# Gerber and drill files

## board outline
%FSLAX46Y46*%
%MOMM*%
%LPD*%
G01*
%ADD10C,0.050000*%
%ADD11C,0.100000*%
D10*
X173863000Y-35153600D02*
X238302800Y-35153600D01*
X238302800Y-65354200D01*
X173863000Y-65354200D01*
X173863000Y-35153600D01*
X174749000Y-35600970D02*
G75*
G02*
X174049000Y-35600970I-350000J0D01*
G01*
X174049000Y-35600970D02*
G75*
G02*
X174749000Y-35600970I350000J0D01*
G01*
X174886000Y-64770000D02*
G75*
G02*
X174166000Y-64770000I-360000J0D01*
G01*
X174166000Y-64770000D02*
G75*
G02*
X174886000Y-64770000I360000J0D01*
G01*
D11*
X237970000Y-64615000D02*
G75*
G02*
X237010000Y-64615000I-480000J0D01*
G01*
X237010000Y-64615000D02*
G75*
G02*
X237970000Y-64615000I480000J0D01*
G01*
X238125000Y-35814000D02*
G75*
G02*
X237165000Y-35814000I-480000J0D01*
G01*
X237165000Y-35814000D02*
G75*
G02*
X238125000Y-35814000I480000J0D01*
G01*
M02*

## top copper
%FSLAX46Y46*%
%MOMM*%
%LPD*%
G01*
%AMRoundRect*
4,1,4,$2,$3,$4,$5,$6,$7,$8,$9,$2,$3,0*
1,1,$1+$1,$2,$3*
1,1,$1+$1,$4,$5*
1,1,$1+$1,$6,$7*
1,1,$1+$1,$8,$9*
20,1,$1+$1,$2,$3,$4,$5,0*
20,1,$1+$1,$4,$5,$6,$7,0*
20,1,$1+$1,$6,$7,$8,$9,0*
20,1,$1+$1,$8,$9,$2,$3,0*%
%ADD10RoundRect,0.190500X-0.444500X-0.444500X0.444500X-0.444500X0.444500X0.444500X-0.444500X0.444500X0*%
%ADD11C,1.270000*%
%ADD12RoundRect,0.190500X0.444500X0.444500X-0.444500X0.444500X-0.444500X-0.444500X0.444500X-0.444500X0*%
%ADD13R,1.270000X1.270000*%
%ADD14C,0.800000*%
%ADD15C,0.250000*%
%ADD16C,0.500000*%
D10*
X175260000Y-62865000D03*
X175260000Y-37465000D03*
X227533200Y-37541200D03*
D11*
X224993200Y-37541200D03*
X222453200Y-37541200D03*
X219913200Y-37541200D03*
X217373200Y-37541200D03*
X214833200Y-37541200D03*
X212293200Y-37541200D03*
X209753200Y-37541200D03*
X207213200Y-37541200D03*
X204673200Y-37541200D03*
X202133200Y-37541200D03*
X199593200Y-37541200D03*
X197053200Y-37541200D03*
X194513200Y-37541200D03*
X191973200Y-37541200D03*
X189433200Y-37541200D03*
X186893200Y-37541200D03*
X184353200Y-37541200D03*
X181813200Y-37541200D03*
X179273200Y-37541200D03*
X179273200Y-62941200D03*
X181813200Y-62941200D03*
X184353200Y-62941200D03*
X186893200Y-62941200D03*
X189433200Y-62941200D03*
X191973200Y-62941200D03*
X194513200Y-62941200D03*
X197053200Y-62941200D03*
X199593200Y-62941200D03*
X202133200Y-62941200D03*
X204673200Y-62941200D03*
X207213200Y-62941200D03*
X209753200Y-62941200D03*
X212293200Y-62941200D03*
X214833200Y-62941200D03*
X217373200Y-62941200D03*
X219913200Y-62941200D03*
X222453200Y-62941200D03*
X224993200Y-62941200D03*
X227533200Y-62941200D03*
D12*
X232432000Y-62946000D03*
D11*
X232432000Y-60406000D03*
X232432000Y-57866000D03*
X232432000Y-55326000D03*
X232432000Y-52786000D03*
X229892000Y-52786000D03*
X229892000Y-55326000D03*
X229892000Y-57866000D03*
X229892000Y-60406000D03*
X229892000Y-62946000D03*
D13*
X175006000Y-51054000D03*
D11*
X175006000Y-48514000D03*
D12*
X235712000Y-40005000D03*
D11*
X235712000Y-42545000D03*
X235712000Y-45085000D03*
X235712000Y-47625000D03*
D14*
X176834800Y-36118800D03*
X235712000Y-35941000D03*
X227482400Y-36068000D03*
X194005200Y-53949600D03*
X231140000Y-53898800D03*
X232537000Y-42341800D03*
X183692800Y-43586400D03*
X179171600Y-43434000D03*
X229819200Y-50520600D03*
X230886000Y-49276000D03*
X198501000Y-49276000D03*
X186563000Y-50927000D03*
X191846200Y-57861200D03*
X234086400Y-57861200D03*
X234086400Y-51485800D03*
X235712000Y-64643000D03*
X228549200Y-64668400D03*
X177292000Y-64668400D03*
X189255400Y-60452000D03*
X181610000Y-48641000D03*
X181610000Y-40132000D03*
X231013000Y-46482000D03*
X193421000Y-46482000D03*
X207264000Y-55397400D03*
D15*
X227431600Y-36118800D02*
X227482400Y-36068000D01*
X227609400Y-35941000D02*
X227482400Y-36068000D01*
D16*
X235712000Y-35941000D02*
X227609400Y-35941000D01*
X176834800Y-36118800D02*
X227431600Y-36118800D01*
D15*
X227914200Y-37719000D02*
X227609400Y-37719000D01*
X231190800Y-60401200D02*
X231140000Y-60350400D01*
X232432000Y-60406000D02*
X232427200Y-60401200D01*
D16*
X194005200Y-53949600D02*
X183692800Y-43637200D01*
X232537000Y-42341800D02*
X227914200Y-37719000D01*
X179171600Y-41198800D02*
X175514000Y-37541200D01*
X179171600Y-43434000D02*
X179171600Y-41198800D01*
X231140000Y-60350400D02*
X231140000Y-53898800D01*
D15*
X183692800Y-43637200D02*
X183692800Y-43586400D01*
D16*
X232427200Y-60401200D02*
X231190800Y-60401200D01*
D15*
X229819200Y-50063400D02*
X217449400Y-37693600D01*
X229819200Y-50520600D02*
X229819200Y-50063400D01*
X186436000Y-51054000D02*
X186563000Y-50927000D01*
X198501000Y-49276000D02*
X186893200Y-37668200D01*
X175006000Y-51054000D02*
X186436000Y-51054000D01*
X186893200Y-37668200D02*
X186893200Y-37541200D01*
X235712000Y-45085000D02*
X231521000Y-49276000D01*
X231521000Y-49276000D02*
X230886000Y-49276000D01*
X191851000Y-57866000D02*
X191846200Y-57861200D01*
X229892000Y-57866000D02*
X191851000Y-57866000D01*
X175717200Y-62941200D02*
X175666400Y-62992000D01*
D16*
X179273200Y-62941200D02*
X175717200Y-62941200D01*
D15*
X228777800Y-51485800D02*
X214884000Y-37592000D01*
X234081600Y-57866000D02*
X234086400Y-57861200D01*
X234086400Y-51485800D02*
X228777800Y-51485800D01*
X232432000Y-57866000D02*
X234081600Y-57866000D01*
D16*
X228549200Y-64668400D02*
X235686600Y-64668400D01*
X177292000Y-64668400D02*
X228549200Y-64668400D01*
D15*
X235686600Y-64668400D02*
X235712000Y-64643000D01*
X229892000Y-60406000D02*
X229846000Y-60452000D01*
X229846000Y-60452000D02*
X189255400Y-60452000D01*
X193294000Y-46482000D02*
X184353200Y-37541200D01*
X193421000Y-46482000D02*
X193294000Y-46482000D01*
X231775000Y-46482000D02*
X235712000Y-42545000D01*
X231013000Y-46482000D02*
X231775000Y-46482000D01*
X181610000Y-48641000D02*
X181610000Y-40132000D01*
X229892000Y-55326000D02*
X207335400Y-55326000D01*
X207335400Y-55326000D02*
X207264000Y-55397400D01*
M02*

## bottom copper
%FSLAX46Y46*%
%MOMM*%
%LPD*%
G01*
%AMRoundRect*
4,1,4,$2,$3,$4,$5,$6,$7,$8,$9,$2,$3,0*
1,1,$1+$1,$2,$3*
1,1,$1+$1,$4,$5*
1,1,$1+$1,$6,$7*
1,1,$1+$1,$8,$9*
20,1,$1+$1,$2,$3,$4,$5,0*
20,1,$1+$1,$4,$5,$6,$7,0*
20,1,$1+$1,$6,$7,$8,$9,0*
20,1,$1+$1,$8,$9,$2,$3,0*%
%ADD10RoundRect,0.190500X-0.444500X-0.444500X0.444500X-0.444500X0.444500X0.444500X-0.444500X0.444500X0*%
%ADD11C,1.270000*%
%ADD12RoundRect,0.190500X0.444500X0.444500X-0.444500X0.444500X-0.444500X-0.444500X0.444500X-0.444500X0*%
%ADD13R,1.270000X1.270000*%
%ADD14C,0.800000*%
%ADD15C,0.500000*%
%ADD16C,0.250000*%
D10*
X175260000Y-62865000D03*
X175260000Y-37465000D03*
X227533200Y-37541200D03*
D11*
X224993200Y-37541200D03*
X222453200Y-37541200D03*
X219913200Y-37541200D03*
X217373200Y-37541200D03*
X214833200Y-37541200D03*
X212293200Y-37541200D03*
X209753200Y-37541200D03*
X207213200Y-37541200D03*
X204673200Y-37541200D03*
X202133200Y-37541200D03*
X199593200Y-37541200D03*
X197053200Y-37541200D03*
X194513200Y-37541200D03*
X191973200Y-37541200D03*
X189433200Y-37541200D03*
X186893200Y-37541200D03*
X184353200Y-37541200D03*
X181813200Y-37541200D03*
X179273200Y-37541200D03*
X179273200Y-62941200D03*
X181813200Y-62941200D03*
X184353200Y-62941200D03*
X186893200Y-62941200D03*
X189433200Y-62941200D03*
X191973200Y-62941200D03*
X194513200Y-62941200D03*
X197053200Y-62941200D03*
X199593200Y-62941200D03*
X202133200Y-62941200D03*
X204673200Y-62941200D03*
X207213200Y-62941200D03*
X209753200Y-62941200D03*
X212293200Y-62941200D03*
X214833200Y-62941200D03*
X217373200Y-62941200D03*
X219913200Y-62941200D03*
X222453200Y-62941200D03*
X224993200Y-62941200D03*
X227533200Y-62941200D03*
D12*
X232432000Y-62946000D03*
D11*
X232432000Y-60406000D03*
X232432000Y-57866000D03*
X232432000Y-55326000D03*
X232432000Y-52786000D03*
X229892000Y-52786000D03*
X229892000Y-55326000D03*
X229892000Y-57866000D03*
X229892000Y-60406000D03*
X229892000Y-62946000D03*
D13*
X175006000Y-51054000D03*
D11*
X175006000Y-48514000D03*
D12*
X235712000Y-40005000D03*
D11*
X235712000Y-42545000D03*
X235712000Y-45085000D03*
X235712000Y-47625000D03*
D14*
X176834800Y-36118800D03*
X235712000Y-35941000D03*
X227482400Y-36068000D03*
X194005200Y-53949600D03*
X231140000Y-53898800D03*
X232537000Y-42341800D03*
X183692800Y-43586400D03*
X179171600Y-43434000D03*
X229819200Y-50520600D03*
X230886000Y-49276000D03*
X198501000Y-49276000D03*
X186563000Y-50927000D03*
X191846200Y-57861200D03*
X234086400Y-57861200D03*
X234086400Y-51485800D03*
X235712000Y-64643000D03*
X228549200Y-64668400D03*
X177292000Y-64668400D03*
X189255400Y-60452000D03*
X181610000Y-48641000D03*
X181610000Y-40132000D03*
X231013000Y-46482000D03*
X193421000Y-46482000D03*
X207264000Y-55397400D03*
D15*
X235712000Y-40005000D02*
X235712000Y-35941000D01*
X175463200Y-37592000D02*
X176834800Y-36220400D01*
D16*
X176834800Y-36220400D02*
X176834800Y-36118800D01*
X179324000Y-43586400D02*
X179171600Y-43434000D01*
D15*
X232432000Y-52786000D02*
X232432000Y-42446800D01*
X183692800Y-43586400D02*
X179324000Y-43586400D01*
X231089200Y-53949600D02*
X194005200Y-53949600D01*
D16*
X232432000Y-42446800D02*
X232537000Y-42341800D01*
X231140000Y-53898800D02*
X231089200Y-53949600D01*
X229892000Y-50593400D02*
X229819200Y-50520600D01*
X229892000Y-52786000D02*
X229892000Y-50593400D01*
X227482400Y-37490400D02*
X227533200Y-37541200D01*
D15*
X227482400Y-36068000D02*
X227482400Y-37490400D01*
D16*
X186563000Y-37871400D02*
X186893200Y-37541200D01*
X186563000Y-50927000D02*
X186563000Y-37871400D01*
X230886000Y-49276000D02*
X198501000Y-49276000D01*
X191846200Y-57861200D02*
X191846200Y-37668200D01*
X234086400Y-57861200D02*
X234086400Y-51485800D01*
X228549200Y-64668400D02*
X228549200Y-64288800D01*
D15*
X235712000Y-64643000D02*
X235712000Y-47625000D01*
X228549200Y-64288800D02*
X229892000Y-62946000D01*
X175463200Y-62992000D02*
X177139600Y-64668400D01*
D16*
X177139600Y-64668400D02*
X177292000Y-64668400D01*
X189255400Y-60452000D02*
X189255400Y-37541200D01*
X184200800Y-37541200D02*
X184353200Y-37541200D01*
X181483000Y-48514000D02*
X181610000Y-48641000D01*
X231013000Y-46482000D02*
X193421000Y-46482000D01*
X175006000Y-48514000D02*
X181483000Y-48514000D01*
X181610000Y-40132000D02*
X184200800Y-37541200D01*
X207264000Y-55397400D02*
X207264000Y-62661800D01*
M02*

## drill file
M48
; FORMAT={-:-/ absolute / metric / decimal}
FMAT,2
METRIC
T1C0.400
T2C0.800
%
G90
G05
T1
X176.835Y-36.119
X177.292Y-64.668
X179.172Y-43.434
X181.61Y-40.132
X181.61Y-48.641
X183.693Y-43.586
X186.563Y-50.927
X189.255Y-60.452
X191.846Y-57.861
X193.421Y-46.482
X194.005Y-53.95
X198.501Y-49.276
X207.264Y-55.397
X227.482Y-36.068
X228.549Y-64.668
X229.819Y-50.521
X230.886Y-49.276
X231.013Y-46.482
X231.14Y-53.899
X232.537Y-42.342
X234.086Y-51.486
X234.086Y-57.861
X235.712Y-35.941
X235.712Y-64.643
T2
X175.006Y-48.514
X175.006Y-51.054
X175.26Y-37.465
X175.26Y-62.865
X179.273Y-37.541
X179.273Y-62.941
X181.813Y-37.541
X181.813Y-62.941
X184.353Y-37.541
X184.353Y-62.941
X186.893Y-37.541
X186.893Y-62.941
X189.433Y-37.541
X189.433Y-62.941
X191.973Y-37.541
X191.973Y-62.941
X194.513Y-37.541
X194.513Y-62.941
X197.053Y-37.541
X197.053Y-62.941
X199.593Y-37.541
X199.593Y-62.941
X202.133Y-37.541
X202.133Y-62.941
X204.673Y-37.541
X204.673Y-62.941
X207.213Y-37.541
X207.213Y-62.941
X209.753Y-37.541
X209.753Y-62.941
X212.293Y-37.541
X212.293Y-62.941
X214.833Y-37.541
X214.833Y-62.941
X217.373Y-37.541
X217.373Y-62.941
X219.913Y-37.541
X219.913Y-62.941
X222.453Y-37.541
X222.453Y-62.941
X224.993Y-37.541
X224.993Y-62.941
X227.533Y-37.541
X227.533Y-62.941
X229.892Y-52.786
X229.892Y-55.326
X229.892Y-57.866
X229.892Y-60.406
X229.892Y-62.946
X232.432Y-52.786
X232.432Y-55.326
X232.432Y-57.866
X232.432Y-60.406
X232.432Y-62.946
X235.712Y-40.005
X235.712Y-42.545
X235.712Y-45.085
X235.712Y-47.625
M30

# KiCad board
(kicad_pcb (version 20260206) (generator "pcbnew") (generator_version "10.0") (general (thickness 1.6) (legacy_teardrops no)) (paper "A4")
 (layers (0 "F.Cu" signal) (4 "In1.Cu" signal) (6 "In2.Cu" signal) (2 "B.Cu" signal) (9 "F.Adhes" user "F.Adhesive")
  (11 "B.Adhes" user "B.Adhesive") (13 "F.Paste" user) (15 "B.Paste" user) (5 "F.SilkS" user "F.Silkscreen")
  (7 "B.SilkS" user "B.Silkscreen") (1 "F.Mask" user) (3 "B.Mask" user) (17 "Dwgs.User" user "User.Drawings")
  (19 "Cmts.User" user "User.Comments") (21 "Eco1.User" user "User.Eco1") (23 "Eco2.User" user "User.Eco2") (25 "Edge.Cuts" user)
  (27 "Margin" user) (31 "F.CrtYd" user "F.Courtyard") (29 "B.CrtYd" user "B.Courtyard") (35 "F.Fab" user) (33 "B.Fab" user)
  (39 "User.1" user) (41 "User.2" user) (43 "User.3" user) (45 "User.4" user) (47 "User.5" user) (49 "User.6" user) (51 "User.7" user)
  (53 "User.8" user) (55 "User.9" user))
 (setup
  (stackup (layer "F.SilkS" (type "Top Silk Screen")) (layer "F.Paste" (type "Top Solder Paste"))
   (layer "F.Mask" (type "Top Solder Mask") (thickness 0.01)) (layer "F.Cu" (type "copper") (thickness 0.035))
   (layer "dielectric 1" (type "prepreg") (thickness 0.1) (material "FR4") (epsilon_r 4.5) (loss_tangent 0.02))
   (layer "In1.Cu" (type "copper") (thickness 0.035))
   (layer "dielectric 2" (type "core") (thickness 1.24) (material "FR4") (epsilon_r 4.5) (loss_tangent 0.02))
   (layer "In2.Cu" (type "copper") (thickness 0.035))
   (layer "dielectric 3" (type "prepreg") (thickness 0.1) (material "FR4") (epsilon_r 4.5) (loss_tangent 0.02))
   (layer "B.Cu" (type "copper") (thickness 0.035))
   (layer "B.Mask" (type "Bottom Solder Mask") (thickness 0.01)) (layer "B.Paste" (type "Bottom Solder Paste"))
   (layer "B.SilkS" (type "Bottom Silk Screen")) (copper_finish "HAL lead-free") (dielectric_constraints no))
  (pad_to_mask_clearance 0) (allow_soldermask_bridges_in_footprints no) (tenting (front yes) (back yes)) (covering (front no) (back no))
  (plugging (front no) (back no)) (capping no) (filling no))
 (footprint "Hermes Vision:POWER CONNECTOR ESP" (layer "F.Cu") (at 175.26 50.165)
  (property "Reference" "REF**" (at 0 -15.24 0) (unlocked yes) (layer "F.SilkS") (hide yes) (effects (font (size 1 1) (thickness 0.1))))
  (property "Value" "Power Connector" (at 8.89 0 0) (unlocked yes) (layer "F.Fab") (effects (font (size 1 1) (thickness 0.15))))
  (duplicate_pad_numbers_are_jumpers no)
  (pad "1" thru_hole roundrect (at 0 12.7) (size 1.27 1.27) (drill 0.8) (layers "*.Cu" "*.Mask") (remove_unused_layers no)
   (roundrect_rratio 0.15))
  (pad "2" thru_hole roundrect (at 0 -12.7) (size 1.27 1.27) (drill 0.8) (layers "*.Cu" "*.Mask") (remove_unused_layers no)
   (roundrect_rratio 0.15))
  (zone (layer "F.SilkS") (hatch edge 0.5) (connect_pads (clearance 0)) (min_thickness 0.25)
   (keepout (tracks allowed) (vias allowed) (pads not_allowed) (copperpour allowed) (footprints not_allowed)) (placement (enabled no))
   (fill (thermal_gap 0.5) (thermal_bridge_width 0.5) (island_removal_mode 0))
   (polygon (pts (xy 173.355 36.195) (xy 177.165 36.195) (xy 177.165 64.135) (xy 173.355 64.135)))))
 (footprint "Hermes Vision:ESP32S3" (layer "F.Cu") (at 204.6732 50.2412)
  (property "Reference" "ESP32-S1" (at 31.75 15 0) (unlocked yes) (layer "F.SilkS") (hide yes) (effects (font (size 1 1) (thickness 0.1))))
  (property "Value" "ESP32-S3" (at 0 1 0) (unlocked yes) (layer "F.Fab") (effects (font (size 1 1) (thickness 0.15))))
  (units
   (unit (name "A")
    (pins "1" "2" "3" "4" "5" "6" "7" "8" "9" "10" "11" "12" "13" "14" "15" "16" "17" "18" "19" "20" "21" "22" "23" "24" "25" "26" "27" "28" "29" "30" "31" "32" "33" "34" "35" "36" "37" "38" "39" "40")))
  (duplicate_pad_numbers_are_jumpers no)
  (pad "1" thru_hole roundrect (at 22.86 -12.7) (size 1.27 1.27) (drill 0.8) (layers "*.Cu" "*.Mask") (remove_unused_layers no)
   (roundrect_rratio 0.15) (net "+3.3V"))
  (pad "2" thru_hole circle (at 20.32 -12.7) (size 1.27 1.27) (drill 0.8) (layers "*.Cu" "*.Mask") (remove_unused_layers no)
   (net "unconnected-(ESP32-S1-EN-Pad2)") (thermal_bridge_angle 90))
  (pad "3" thru_hole circle (at 17.78 -12.7) (size 1.27 1.27) (drill 0.8) (layers "*.Cu" "*.Mask") (remove_unused_layers no)
   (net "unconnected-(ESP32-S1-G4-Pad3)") (thermal_bridge_angle 90))
  (pad "4" thru_hole circle (at 15.24 -12.7) (size 1.27 1.27) (drill 0.8) (layers "*.Cu" "*.Mask") (remove_unused_layers no)
   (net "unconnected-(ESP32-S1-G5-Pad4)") (thermal_bridge_angle 90))
  (pad "5" thru_hole circle (at 12.7 -12.7) (size 1.27 1.27) (drill 0.8) (layers "*.Cu" "*.Mask") (remove_unused_layers no)
   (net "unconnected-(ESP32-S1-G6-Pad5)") (thermal_bridge_angle 90))
  (pad "6" thru_hole circle (at 10.16 -12.7) (size 1.27 1.27) (drill 0.8) (layers "*.Cu" "*.Mask") (remove_unused_layers no)
   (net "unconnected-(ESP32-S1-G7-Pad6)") (thermal_bridge_angle 90))
  (pad "7" thru_hole circle (at 7.62 -12.7) (size 1.27 1.27) (drill 0.8) (layers "*.Cu" "*.Mask") (remove_unused_layers no)
   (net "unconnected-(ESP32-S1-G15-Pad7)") (thermal_bridge_angle 90))
  (pad "8" thru_hole circle (at 5.08 -12.7) (size 1.27 1.27) (drill 0.8) (layers "*.Cu" "*.Mask") (remove_unused_layers no)
   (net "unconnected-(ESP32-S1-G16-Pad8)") (thermal_bridge_angle 90))
  (pad "9" thru_hole circle (at 2.54 -12.7) (size 1.27 1.27) (drill 0.8) (layers "*.Cu" "*.Mask") (remove_unused_layers no)
   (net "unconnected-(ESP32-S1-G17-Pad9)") (thermal_bridge_angle 90))
  (pad "10" thru_hole circle (at 0 -12.7) (size 1.27 1.27) (drill 0.8) (layers "*.Cu" "*.Mask") (remove_unused_layers no)
   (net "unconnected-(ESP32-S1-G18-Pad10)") (thermal_bridge_angle 90))
  (pad "11" thru_hole circle (at -2.54 -12.7) (size 1.27 1.27) (drill 0.8) (layers "*.Cu" "*.Mask") (remove_unused_layers no)
   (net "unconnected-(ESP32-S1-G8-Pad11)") (thermal_bridge_angle 90))
  (pad "12" thru_hole circle (at -5.08 -12.7) (size 1.27 1.27) (drill 0.8) (layers "*.Cu" "*.Mask") (remove_unused_layers no)
   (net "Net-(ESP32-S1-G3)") (thermal_bridge_angle 90))
  (pad "13" thru_hole circle (at -7.62 -12.7) (size 1.27 1.27) (drill 0.8) (layers "*.Cu" "*.Mask") (remove_unused_layers no)
   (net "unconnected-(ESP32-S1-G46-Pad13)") (thermal_bridge_angle 90))
  (pad "14" thru_hole circle (at -10.16 -12.7) (size 1.27 1.27) (drill 0.8) (layers "*.Cu" "*.Mask") (remove_unused_layers no)
   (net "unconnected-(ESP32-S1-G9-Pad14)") (thermal_bridge_angle 90))
  (pad "15" thru_hole circle (at -12.7 -12.7) (size 1.27 1.27) (drill 0.8) (layers "*.Cu" "*.Mask") (remove_unused_layers no)
   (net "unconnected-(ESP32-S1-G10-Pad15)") (thermal_bridge_angle 90))
  (pad "16" thru_hole circle (at -15.24 -12.7) (size 1.27 1.27) (drill 0.8) (layers "*.Cu" "*.Mask") (remove_unused_layers no)
   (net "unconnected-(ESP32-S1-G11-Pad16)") (thermal_bridge_angle 90))
  (pad "17" thru_hole circle (at -17.78 -12.7) (size 1.27 1.27) (drill 0.8) (layers "*.Cu" "*.Mask") (remove_unused_layers no)
   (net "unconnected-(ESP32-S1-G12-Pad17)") (thermal_bridge_angle 90))
  (pad "18" thru_hole circle (at -20.32 -12.7) (size 1.27 1.27) (drill 0.8) (layers "*.Cu" "*.Mask") (remove_unused_layers no)
   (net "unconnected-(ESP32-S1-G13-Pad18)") (thermal_bridge_angle 90))
  (pad "19" thru_hole circle (at -22.86 -12.7) (size 1.27 1.27) (drill 0.8) (layers "*.Cu" "*.Mask") (remove_unused_layers no)
   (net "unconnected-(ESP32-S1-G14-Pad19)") (thermal_bridge_angle 90))
  (pad "20" thru_hole circle (at -25.4 -12.7) (size 1.27 1.27) (drill 0.8) (layers "*.Cu" "*.Mask") (remove_unused_layers no)
   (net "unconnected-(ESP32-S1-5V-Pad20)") (thermal_bridge_angle 90))
  (pad "21" thru_hole circle (at -25.4 12.7) (size 1.27 1.27) (drill 0.8) (layers "*.Cu" "*.Mask") (remove_unused_layers no)
   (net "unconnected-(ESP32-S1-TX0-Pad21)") (thermal_bridge_angle 90))
  (pad "22" thru_hole circle (at -22.86 12.7) (size 1.27 1.27) (drill 0.8) (layers "*.Cu" "*.Mask") (remove_unused_layers no)
   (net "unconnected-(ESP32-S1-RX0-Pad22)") (thermal_bridge_angle 90))
  (pad "23" thru_hole circle (at -20.32 12.7) (size 1.27 1.27) (drill 0.8) (layers "*.Cu" "*.Mask") (remove_unused_layers no)
   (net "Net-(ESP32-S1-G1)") (thermal_bridge_angle 90))
  (pad "24" thru_hole circle (at -17.78 12.7) (size 1.27 1.27) (drill 0.8) (layers "*.Cu" "*.Mask") (remove_unused_layers no)
   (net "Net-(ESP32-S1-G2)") (thermal_bridge_angle 90))
  (pad "25" thru_hole circle (at -15.24 12.7) (size 1.27 1.27) (drill 0.8) (layers "*.Cu" "*.Mask") (remove_unused_layers no)
   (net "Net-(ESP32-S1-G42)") (thermal_bridge_angle 90))
  (pad "26" thru_hole circle (at -12.7 12.7) (size 1.27 1.27) (drill 0.8) (layers "*.Cu" "*.Mask") (remove_unused_layers no)
   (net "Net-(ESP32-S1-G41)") (thermal_bridge_angle 90))
  (pad "27" thru_hole circle (at -10.16 12.7) (size 1.27 1.27) (drill 0.8) (layers "*.Cu" "*.Mask") (remove_unused_layers no)
   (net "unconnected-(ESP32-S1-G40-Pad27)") (thermal_bridge_angle 90))
  (pad "28" thru_hole circle (at -7.62 12.7) (size 1.27 1.27) (drill 0.8) (layers "*.Cu" "*.Mask") (remove_unused_layers no)
   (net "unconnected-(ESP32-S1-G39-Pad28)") (thermal_bridge_angle 90))
  (pad "29" thru_hole circle (at -5.08 12.7) (size 1.27 1.27) (drill 0.8) (layers "*.Cu" "*.Mask") (remove_unused_layers no)
   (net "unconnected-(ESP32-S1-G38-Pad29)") (thermal_bridge_angle 90))
  (pad "30" thru_hole circle (at -2.54 12.7) (size 1.27 1.27) (drill 0.8) (layers "*.Cu" "*.Mask") (remove_unused_layers no)
   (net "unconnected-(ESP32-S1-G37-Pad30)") (thermal_bridge_angle 90))
  (pad "31" thru_hole circle (at 0 12.7) (size 1.27 1.27) (drill 0.8) (layers "*.Cu" "*.Mask") (remove_unused_layers no)
   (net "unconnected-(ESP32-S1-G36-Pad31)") (thermal_bridge_angle 90))
  (pad "32" thru_hole circle (at 2.54 12.7) (size 1.27 1.27) (drill 0.8) (layers "*.Cu" "*.Mask") (remove_unused_layers no)
   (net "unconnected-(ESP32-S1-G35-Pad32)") (thermal_bridge_angle 90))
  (pad "33" thru_hole circle (at 5.08 12.7) (size 1.27 1.27) (drill 0.8) (layers "*.Cu" "*.Mask") (remove_unused_layers no)
   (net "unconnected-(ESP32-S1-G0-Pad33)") (thermal_bridge_angle 90))
  (pad "34" thru_hole circle (at 7.62 12.7) (size 1.27 1.27) (drill 0.8) (layers "*.Cu" "*.Mask") (remove_unused_layers no)
   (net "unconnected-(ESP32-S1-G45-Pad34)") (thermal_bridge_angle 90))
  (pad "35" thru_hole circle (at 10.16 12.7) (size 1.27 1.27) (drill 0.8) (layers "*.Cu" "*.Mask") (remove_unused_layers no)
   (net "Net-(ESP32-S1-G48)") (thermal_bridge_angle 90))
  (pad "36" thru_hole circle (at 12.7 12.7) (size 1.27 1.27) (drill 0.8) (layers "*.Cu" "*.Mask") (remove_unused_layers no)
   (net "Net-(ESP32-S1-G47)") (thermal_bridge_angle 90))
  (pad "37" thru_hole circle (at 15.24 12.7) (size 1.27 1.27) (drill 0.8) (layers "*.Cu" "*.Mask") (remove_unused_layers no)
   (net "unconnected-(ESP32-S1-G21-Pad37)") (thermal_bridge_angle 90))
  (pad "38" thru_hole circle (at 17.78 12.7) (size 1.27 1.27) (drill 0.8) (layers "*.Cu" "*.Mask") (remove_unused_layers no)
   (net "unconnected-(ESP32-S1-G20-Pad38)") (thermal_bridge_angle 90))
  (pad "39" thru_hole circle (at 20.32 12.7) (size 1.27 1.27) (drill 0.8) (layers "*.Cu" "*.Mask") (remove_unused_layers no)
   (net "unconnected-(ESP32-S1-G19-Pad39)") (thermal_bridge_angle 90))
  (pad "40" thru_hole circle (at 22.86 12.7) (size 1.27 1.27) (drill 0.8) (layers "*.Cu" "*.Mask") (remove_unused_layers no) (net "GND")
   (thermal_bridge_angle 90))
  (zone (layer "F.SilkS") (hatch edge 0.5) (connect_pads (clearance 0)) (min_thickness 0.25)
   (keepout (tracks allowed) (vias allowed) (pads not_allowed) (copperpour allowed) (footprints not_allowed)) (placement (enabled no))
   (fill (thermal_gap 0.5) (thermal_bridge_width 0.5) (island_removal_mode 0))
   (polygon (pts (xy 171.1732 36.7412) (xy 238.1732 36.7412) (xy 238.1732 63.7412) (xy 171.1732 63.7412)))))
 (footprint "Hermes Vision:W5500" (layer "B.Cu") (at 205 50.5 180)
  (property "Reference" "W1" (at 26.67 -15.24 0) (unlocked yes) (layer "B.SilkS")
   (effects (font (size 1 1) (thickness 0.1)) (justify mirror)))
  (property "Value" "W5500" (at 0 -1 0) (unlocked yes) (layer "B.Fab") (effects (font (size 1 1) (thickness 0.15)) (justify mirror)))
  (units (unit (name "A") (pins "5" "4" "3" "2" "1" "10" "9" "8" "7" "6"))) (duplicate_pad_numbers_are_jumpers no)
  (pad "1" thru_hole roundrect (at -27.432 -12.446 180) (size 1.27 1.27) (drill 0.8) (layers "*.Cu" "*.Mask") (remove_unused_layers no)
   (roundrect_rratio 0.15) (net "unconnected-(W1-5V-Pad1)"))
  (pad "2" thru_hole circle (at -27.432 -9.906 180) (size 1.27 1.27) (drill 0.8) (layers "*.Cu" "*.Mask") (remove_unused_layers no)
   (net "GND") (thermal_bridge_angle 90))
  (pad "3" thru_hole circle (at -27.432 -7.366 180) (size 1.27 1.27) (drill 0.8) (layers "*.Cu" "*.Mask") (remove_unused_layers no)
   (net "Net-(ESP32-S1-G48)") (thermal_bridge_angle 90))
  (pad "4" thru_hole circle (at -27.432 -4.826 180) (size 1.27 1.27) (drill 0.8) (layers "*.Cu" "*.Mask") (remove_unused_layers no)
   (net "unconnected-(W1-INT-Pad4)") (thermal_bridge_angle 90))
  (pad "5" thru_hole circle (at -27.432 -2.286 180) (size 1.27 1.27) (drill 0.8) (layers "*.Cu" "*.Mask") (remove_unused_layers no)
   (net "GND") (thermal_bridge_angle 90))
  (pad "6" thru_hole circle (at -24.892 -2.286 180) (size 1.27 1.27) (drill 0.8) (layers "*.Cu" "*.Mask") (remove_unused_layers no)
   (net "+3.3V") (thermal_bridge_angle 90))
  (pad "7" thru_hole circle (at -24.892 -4.826 180) (size 1.27 1.27) (drill 0.8) (layers "*.Cu" "*.Mask") (remove_unused_layers no)
   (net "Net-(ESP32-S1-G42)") (thermal_bridge_angle 90))
  (pad "8" thru_hole circle (at -24.892 -7.366 180) (size 1.27 1.27) (drill 0.8) (layers "*.Cu" "*.Mask") (remove_unused_layers no)
   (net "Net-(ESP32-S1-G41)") (thermal_bridge_angle 90))
  (pad "9" thru_hole circle (at -24.892 -9.906 180) (size 1.27 1.27) (drill 0.8) (layers "*.Cu" "*.Mask") (remove_unused_layers no)
   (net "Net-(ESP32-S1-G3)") (thermal_bridge_angle 90))
  (pad "10" thru_hole circle (at -24.892 -12.446 180) (size 1.27 1.27) (drill 0.8) (layers "*.Cu" "*.Mask") (remove_unused_layers no)
   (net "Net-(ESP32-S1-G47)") (thermal_bridge_angle 90))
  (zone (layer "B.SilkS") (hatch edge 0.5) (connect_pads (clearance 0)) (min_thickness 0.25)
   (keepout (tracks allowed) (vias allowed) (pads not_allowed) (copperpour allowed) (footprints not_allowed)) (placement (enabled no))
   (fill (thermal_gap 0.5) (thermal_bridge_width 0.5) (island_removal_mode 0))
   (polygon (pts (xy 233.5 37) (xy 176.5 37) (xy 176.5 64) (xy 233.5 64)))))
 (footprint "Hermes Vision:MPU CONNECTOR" (layer "B.Cu") (at 174.879 49.53 180)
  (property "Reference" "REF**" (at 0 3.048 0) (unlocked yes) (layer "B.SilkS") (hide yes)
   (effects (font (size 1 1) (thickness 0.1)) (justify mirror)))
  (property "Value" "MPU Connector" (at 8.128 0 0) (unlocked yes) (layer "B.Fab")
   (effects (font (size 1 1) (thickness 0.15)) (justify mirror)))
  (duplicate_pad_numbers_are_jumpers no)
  (pad "1" thru_hole rect (at -0.127 -1.524 180) (size 1.27 1.27) (drill 0.8) (layers "*.Cu" "*.Mask") (remove_unused_layers no))
  (pad "2" thru_hole circle (at -0.127 1.016 180) (size 1.27 1.27) (drill 0.8) (layers "*.Cu" "*.Mask") (remove_unused_layers no)
   (thermal_bridge_angle 90))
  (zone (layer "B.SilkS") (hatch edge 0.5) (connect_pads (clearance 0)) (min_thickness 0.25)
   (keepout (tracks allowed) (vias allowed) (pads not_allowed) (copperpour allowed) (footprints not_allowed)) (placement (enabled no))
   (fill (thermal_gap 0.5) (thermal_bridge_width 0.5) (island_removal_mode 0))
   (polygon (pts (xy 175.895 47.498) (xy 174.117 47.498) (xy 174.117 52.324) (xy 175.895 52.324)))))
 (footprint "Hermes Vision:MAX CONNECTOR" (layer "B.Cu") (at 235.712 44.069 180)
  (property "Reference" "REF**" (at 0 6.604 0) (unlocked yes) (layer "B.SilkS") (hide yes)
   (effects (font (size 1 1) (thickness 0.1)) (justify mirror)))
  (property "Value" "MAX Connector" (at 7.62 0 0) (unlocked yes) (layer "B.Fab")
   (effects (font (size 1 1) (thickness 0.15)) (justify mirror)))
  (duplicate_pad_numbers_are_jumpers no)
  (pad "1" thru_hole roundrect (at 0 4.064 180) (size 1.27 1.27) (drill 0.8) (layers "*.Cu" "*.Mask") (remove_unused_layers no)
   (roundrect_rratio 0.15))
  (pad "2" thru_hole circle (at 0 1.524 180) (size 1.27 1.27) (drill 0.8) (layers "*.Cu" "*.Mask") (remove_unused_layers no)
   (thermal_bridge_angle 90))
  (pad "3" thru_hole circle (at 0 -1.016 180) (size 1.27 1.27) (drill 0.8) (layers "*.Cu" "*.Mask") (remove_unused_layers no)
   (thermal_bridge_angle 90))
  (pad "4" thru_hole circle (at 0 -3.556 180) (size 1.27 1.27) (drill 0.8) (layers "*.Cu" "*.Mask") (remove_unused_layers no)
   (thermal_bridge_angle 90))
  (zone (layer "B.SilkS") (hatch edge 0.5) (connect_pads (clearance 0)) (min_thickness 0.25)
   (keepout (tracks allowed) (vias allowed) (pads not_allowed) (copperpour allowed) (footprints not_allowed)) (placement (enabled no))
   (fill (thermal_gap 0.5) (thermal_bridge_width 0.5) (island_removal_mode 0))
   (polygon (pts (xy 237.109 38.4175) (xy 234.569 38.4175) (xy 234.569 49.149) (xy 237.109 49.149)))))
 (gr_rect (start 173.863 35.1536) (end 238.3028 65.3542) (stroke (width 0.05) (type default)) (fill no) (layer "Edge.Cuts"))
 (gr_circle (center 174.399 35.60097) (end 174.749 35.60097) (stroke (width 0.05) (type default)) (fill no) (layer "Edge.Cuts"))
 (gr_circle (center 174.526 64.77) (end 174.886 64.77) (stroke (width 0.05) (type default)) (fill no) (layer "Edge.Cuts"))
 (gr_circle (center 237.49 64.615) (end 237.97 64.615) (stroke (width 0) (type default)) (fill no) (layer "Edge.Cuts"))
 (gr_circle (center 237.645 35.814) (end 238.125 35.814) (stroke (width 0) (type default)) (fill no) (layer "Edge.Cuts"))
 (segment (start 227.4316 36.1188) (end 227.4824 36.068) (width 0.25) (layer "F.Cu") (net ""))
 (segment (start 227.6094 35.941) (end 227.4824 36.068) (width 0.25) (layer "F.Cu") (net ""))
 (segment (start 235.712 35.941) (end 227.6094 35.941) (width 0.5) (layer "F.Cu") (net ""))
 (segment (start 176.8348 36.1188) (end 227.4316 36.1188) (width 0.5) (layer "F.Cu") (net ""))
 (via (at 176.8348 36.1188) (size 0.8) (drill 0.4) (layers "F.Cu" "B.Cu") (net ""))
 (via (at 235.712 35.941) (size 0.8) (drill 0.4) (layers "F.Cu" "B.Cu") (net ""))
 (via (at 227.4824 36.068) (size 0.8) (drill 0.4) (layers "F.Cu" "B.Cu") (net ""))
 (segment (start 235.712 40.005) (end 235.712 35.941) (width 0.5) (layer "B.Cu") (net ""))
 (segment (start 175.4632 37.592) (end 176.8348 36.2204) (width 0.5) (layer "B.Cu") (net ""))
 (segment (start 176.8348 36.2204) (end 176.8348 36.1188) (width 0.25) (layer "B.Cu") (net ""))
 (segment (start 227.9142 37.719) (end 227.6094 37.719) (width 0.25) (layer "F.Cu") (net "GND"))
 (segment (start 231.1908 60.4012) (end 231.14 60.3504) (width 0.25) (layer "F.Cu") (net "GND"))
 (segment (start 232.432 60.406) (end 232.4272 60.4012) (width 0.25) (layer "F.Cu") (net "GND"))
 (segment (start 194.0052 53.9496) (end 183.6928 43.6372) (width 0.5) (layer "F.Cu") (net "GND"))
 (segment (start 232.537 42.3418) (end 227.9142 37.719) (width 0.5) (layer "F.Cu") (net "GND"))
 (segment (start 179.1716 41.1988) (end 175.514 37.5412) (width 0.5) (layer "F.Cu") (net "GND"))
 (segment (start 179.1716 43.434) (end 179.1716 41.1988) (width 0.5) (layer "F.Cu") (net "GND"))
 (segment (start 231.14 60.3504) (end 231.14 53.8988) (width 0.5) (layer "F.Cu") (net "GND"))
 (segment (start 183.6928 43.6372) (end 183.6928 43.5864) (width 0.25) (layer "F.Cu") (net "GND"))
 (segment (start 232.4272 60.4012) (end 231.1908 60.4012) (width 0.5) (layer "F.Cu") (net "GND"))
 (via (at 194.0052 53.9496) (size 0.8) (drill 0.4) (layers "F.Cu" "B.Cu") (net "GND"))
 (via (at 231.14 53.8988) (size 0.8) (drill 0.4) (layers "F.Cu" "B.Cu") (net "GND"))
 (via (at 232.537 42.3418) (size 0.8) (drill 0.4) (layers "F.Cu" "B.Cu") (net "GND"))
 (via (at 183.6928 43.5864) (size 0.8) (drill 0.4) (layers "F.Cu" "B.Cu") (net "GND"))
 (via (at 179.1716 43.434) (size 0.8) (drill 0.4) (layers "F.Cu" "B.Cu") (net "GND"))
 (segment (start 179.324 43.5864) (end 179.1716 43.434) (width 0.25) (layer "B.Cu") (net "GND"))
 (segment (start 232.432 52.786) (end 232.432 42.4468) (width 0.5) (layer "B.Cu") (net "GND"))
 (segment (start 183.6928 43.5864) (end 179.324 43.5864) (width 0.5) (layer "B.Cu") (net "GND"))
 (segment (start 231.0892 53.9496) (end 194.0052 53.9496) (width 0.5) (layer "B.Cu") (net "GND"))
 (segment (start 232.432 42.4468) (end 232.537 42.3418) (width 0.25) (layer "B.Cu") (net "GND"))
 (segment (start 231.14 53.8988) (end 231.0892 53.9496) (width 0.25) (layer "B.Cu") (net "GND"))
 (segment (start 229.8192 50.0634) (end 217.4494 37.6936) (width 0.25) (layer "F.Cu") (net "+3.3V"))
 (segment (start 229.8192 50.5206) (end 229.8192 50.0634) (width 0.25) (layer "F.Cu") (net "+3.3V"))
 (via (at 229.8192 50.5206) (size 0.8) (drill 0.4) (layers "F.Cu" "B.Cu") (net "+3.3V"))
 (segment (start 229.892 50.5934) (end 229.8192 50.5206) (width 0.25) (layer "B.Cu") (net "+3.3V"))
 (segment (start 229.892 52.786) (end 229.892 50.5934) (width 0.25) (layer "B.Cu") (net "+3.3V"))
 (segment (start 227.4824 37.4904) (end 227.5332 37.5412) (width 0.25) (layer "B.Cu") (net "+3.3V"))
 (segment (start 227.4824 36.068) (end 227.4824 37.4904) (width 0.5) (layer "B.Cu") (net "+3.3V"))
 (segment (start 186.436 51.054) (end 186.563 50.927) (width 0.25) (layer "F.Cu") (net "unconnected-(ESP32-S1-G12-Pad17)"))
 (segment (start 198.501 49.276) (end 186.8932 37.6682) (width 0.25) (layer "F.Cu") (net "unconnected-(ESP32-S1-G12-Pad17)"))
 (segment (start 175.006 51.054) (end 186.436 51.054) (width 0.25) (layer "F.Cu") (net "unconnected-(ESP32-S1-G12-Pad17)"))
 (segment (start 186.8932 37.6682) (end 186.8932 37.5412) (width 0.25) (layer "F.Cu") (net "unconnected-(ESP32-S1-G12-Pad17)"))
 (segment (start 235.712 45.085) (end 231.521 49.276) (width 0.25) (layer "F.Cu") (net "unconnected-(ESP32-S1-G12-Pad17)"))
 (segment (start 231.521 49.276) (end 230.886 49.276) (width 0.25) (layer "F.Cu") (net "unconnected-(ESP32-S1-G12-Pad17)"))
 (via (at 230.886 49.276) (size 0.8) (drill 0.4) (layers "F.Cu" "B.Cu") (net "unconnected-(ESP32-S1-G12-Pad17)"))
 (via (at 198.501 49.276) (size 0.8) (drill 0.4) (layers "F.Cu" "B.Cu") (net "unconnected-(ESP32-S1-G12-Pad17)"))
 (via (at 186.563 50.927) (size 0.8) (drill 0.4) (layers "F.Cu" "B.Cu") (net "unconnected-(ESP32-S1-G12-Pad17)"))
 (segment (start 186.563 37.8714) (end 186.8932 37.5412) (width 0.25) (layer "B.Cu") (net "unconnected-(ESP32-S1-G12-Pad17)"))
 (segment (start 186.563 50.927) (end 186.563 37.8714) (width 0.25) (layer "B.Cu") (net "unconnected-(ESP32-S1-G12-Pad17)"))
 (segment (start 230.886 49.276) (end 198.501 49.276) (width 0.25) (layer "B.Cu") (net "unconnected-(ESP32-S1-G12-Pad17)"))
 (segment (start 191.851 57.866) (end 191.8462 57.8612) (width 0.25) (layer "F.Cu") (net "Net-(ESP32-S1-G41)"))
 (segment (start 229.892 57.866) (end 191.851 57.866) (width 0.25) (layer "F.Cu") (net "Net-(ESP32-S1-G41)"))
 (via (at 191.8462 57.8612) (size 0.8) (drill 0.4) (layers "F.Cu" "B.Cu") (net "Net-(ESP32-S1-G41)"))
 (segment (start 191.8462 57.8612) (end 191.8462 37.6682) (width 0.25) (layer "B.Cu") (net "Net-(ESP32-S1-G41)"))
 (segment (start 175.7172 62.9412) (end 175.6664 62.992) (width 0.25) (layer "F.Cu") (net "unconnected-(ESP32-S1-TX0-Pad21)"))
 (segment (start 179.2732 62.9412) (end 175.7172 62.9412) (width 0.5) (layer "F.Cu") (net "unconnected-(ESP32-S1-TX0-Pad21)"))
 (segment (start 228.7778 51.4858) (end 214.884 37.592) (width 0.25) (layer "F.Cu") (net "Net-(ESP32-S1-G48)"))
 (segment (start 234.0816 57.866) (end 234.0864 57.8612) (width 0.25) (layer "F.Cu") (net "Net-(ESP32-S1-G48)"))
 (segment (start 234.0864 51.4858) (end 228.7778 51.4858) (width 0.25) (layer "F.Cu") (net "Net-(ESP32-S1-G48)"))
 (segment (start 232.432 57.866) (end 234.0816 57.866) (width 0.25) (layer "F.Cu") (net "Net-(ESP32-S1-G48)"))
 (via (at 234.0864 57.8612) (size 0.8) (drill 0.4) (layers "F.Cu" "B.Cu") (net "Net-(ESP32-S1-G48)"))
 (via (at 234.0864 51.4858) (size 0.8) (drill 0.4) (layers "F.Cu" "B.Cu") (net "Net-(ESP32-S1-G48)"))
 (segment (start 234.0864 57.8612) (end 234.0864 51.4858) (width 0.25) (layer "B.Cu") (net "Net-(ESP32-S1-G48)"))
 (segment (start 228.5492 64.6684) (end 235.6866 64.6684) (width 0.5) (layer "F.Cu") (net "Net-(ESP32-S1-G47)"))
 (segment (start 177.292 64.6684) (end 228.5492 64.6684) (width 0.5) (layer "F.Cu") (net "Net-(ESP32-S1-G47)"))
 (segment (start 235.6866 64.6684) (end 235.712 64.643) (width 0.25) (layer "F.Cu") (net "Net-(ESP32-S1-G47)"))
 (via (at 235.712 64.643) (size 0.8) (drill 0.4) (layers "F.Cu" "B.Cu") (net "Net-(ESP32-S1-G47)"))
 (via (at 228.5492 64.6684) (size 0.8) (drill 0.4) (layers "F.Cu" "B.Cu") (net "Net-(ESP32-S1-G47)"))
 (via (at 177.292 64.6684) (size 0.8) (drill 0.4) (layers "F.Cu" "B.Cu") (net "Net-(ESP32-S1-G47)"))
 (segment (start 228.5492 64.6684) (end 228.5492 64.2888) (width 0.25) (layer "B.Cu") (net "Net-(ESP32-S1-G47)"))
 (segment (start 235.712 64.643) (end 235.712 47.625) (width 0.5) (layer "B.Cu") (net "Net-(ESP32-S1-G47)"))
 (segment (start 228.5492 64.2888) (end 229.892 62.946) (width 0.5) (layer "B.Cu") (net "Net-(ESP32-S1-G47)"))
 (segment (start 175.4632 62.992) (end 177.1396 64.6684) (width 0.5) (layer "B.Cu") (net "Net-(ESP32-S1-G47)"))
 (segment (start 177.1396 64.6684) (end 177.292 64.6684) (width 0.25) (layer "B.Cu") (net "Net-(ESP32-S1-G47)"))
 (segment (start 229.892 60.406) (end 229.846 60.452) (width 0.25) (layer "F.Cu") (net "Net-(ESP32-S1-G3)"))
 (segment (start 229.846 60.452) (end 189.2554 60.452) (width 0.25) (layer "F.Cu") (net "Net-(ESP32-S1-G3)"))
 (via (at 189.2554 60.452) (size 0.8) (drill 0.4) (layers "F.Cu" "B.Cu") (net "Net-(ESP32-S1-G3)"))
 (segment (start 189.2554 60.452) (end 189.2554 37.5412) (width 0.25) (layer "B.Cu") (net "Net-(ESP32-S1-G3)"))
 (segment (start 193.294 46.482) (end 184.3532 37.5412) (width 0.25) (layer "F.Cu") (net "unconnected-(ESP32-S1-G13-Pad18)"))
 (segment (start 193.421 46.482) (end 193.294 46.482) (width 0.25) (layer "F.Cu") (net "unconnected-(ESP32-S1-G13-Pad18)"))
 (segment (start 231.775 46.482) (end 235.712 42.545) (width 0.25) (layer "F.Cu") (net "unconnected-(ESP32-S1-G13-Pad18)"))
 (segment (start 231.013 46.482) (end 231.775 46.482) (width 0.25) (layer "F.Cu") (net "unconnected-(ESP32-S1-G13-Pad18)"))
 (segment (start 181.61 48.641) (end 181.61 40.132) (width 0.25) (layer "F.Cu") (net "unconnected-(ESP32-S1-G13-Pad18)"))
 (via (at 181.61 48.641) (size 0.8) (drill 0.4) (layers "F.Cu" "B.Cu") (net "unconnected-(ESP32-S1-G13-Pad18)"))
 (via (at 181.61 40.132) (size 0.8) (drill 0.4) (layers "F.Cu" "B.Cu") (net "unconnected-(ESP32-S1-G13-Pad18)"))
 (via (at 231.013 46.482) (size 0.8) (drill 0.4) (layers "F.Cu" "B.Cu") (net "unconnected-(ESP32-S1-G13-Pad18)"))
 (via (at 193.421 46.482) (size 0.8) (drill 0.4) (layers "F.Cu" "B.Cu") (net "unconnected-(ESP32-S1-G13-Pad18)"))
 (segment (start 184.2008 37.5412) (end 184.3532 37.5412) (width 0.25) (layer "B.Cu") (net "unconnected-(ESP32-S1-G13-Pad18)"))
 (segment (start 181.483 48.514) (end 181.61 48.641) (width 0.25) (layer "B.Cu") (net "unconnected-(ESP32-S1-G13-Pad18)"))
 (segment (start 231.013 46.482) (end 193.421 46.482) (width 0.25) (layer "B.Cu") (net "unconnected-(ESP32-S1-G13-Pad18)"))
 (segment (start 175.006 48.514) (end 181.483 48.514) (width 0.25) (layer "B.Cu") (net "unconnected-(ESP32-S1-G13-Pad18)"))
 (segment (start 181.61 40.132) (end 184.2008 37.5412) (width 0.25) (layer "B.Cu") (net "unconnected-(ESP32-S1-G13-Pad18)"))
 (segment (start 229.892 55.326) (end 207.3354 55.326) (width 0.25) (layer "F.Cu") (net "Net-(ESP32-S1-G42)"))
 (segment (start 207.3354 55.326) (end 207.264 55.3974) (width 0.25) (layer "F.Cu") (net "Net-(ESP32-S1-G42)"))
 (via (at 207.264 55.3974) (size 0.8) (drill 0.4) (layers "F.Cu" "B.Cu") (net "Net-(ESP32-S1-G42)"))
 (segment (start 207.264 55.3974) (end 207.264 62.6618) (width 0.25) (layer "B.Cu") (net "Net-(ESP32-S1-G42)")))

